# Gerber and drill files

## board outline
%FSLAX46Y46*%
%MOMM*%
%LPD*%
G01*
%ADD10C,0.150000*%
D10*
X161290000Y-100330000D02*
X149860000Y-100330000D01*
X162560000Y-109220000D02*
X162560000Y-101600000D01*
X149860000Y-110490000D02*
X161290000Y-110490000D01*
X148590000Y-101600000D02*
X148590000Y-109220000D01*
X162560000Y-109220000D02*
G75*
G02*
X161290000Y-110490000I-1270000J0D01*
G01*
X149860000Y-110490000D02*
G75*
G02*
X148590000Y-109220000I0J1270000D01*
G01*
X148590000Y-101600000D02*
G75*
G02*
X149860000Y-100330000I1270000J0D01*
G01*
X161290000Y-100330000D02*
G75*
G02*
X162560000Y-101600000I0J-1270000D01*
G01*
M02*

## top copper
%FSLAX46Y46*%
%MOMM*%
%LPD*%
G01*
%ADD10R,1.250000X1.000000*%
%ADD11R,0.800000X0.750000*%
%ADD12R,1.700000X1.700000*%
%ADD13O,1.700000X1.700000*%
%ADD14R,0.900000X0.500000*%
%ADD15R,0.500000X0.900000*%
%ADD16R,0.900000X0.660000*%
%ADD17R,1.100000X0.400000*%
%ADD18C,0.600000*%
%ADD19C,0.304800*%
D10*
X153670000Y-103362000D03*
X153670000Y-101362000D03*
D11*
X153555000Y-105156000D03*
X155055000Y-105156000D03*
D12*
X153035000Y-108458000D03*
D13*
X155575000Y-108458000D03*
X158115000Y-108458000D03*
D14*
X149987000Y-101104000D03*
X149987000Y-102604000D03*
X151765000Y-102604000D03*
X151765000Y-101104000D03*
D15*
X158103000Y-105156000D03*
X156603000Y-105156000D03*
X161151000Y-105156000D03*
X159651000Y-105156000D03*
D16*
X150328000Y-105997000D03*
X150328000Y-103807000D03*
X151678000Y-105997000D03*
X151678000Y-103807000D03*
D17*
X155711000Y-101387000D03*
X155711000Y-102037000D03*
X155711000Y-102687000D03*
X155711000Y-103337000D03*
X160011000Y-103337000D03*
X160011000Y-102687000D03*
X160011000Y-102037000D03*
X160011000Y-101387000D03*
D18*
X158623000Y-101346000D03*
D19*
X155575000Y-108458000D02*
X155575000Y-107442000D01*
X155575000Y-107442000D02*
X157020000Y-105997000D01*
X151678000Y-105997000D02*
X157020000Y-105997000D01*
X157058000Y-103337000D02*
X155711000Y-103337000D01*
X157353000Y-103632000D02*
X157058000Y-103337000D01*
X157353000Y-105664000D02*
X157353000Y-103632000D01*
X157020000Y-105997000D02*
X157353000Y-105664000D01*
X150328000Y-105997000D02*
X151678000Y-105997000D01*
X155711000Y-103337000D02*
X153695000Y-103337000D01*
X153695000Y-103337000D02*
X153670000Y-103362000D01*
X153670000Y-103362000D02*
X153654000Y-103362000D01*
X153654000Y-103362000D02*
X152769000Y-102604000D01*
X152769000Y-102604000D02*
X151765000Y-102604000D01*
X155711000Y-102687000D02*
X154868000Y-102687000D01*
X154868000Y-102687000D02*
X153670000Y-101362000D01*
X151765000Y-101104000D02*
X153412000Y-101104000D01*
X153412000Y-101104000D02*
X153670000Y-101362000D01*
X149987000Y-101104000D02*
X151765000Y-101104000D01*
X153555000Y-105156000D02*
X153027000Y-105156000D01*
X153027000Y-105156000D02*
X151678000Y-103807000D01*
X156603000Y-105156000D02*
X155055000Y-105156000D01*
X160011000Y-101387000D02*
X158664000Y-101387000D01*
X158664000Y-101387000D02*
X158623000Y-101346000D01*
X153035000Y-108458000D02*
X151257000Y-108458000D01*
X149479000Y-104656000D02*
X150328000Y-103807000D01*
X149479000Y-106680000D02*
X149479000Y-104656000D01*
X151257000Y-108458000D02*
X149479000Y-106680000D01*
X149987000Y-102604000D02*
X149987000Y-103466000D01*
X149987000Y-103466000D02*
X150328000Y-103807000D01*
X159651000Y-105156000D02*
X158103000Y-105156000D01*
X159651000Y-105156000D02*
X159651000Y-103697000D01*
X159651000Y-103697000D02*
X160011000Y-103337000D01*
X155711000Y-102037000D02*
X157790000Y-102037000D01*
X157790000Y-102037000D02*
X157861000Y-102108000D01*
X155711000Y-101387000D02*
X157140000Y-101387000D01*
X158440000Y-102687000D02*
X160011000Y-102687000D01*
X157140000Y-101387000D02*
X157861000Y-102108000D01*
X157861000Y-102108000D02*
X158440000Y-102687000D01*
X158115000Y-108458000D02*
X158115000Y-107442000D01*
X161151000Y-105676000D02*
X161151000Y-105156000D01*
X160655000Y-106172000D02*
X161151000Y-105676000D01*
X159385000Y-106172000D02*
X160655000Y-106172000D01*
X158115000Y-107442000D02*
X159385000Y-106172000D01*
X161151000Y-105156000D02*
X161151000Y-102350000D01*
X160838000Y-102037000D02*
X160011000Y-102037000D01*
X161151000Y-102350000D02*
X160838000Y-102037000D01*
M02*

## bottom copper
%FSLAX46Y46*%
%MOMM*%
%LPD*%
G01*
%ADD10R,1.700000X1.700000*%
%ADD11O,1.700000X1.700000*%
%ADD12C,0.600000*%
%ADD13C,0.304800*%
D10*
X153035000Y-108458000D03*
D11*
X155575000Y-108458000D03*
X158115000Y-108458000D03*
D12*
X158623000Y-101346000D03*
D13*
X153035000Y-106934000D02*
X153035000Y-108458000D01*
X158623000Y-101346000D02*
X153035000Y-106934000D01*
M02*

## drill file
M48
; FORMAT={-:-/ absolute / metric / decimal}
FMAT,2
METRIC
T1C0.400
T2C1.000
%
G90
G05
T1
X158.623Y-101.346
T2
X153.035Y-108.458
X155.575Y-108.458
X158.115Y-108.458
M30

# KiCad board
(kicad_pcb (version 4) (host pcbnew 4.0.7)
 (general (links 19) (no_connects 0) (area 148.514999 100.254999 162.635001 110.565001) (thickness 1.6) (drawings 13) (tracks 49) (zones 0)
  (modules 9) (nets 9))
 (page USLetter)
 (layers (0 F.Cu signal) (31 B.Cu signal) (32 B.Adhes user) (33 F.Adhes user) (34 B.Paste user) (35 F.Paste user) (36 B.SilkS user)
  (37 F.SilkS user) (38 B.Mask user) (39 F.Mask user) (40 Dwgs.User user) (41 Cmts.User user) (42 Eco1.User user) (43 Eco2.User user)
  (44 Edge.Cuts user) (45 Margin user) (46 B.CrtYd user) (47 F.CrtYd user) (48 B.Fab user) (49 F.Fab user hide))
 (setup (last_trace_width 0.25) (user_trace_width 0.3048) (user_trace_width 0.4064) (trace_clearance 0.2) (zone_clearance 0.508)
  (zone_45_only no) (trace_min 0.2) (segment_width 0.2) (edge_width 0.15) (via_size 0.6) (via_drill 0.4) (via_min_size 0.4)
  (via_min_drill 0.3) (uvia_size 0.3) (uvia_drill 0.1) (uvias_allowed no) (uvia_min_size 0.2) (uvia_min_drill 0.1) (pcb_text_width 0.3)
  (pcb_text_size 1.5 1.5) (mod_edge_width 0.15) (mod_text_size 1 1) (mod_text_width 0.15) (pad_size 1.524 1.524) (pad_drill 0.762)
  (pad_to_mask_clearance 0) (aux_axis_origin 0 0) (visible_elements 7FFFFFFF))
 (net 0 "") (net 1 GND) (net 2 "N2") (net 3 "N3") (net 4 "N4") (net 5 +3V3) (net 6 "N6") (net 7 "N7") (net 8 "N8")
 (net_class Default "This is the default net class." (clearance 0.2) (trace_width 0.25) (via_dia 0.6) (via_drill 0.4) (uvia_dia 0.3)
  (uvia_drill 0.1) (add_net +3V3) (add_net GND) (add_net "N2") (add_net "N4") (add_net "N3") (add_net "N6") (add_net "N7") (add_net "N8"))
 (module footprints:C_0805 (layer F.Cu) (at 153.67 102.362 90)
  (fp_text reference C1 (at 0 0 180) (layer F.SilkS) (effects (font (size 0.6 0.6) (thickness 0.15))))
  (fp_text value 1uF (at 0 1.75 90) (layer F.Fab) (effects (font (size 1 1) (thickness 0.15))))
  (pad 1 smd rect (at -1 0 90) (size 1 1.25) (layers F.Cu F.Paste F.Mask) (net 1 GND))
  (pad 2 smd rect (at 1 0 90) (size 1 1.25) (layers F.Cu F.Paste F.Mask) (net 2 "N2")))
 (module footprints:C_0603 (layer F.Cu) (at 154.305 105.156 180)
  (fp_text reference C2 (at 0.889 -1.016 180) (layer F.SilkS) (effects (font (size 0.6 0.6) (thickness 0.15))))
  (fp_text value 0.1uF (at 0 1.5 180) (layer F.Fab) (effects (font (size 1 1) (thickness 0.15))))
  (pad 2 smd rect (at 0.75 0 180) (size 0.8 0.75) (layers F.Cu F.Paste F.Mask) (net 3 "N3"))
  (pad 1 smd rect (at -0.75 0 180) (size 0.8 0.75) (layers F.Cu F.Paste F.Mask) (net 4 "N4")))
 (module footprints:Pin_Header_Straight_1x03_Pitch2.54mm (layer F.Cu) (at 153.035 108.458 90)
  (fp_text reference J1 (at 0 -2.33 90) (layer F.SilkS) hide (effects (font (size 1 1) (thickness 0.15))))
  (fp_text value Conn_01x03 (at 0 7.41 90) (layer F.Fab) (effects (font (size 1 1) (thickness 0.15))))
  (pad 1 thru_hole rect (at 0 0 90) (size 1.7 1.7) (drill 1) (layers *.Cu *.Mask) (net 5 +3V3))
  (pad 2 thru_hole oval (at 0 2.54 90) (size 1.7 1.7) (drill 1) (layers *.Cu *.Mask) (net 1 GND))
  (pad 3 thru_hole oval (at 0 5.08 90) (size 1.7 1.7) (drill 1) (layers *.Cu *.Mask) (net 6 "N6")))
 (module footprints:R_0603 (layer F.Cu) (at 149.987 101.854 270)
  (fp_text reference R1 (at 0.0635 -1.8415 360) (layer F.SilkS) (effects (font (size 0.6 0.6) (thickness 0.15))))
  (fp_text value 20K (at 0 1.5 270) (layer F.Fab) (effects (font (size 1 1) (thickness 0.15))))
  (pad 1 smd rect (at -0.75 0 270) (size 0.5 0.9) (layers F.Cu F.Paste F.Mask) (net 2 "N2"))
  (pad 2 smd rect (at 0.75 0 270) (size 0.5 0.9) (layers F.Cu F.Paste F.Mask) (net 5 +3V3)))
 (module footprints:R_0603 (layer F.Cu) (at 151.765 101.854 90)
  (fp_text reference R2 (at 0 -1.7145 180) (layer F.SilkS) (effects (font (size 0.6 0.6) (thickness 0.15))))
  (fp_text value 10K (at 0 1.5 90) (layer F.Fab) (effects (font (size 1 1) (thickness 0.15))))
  (pad 1 smd rect (at -0.75 0 90) (size 0.5 0.9) (layers F.Cu F.Paste F.Mask) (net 1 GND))
  (pad 2 smd rect (at 0.75 0 90) (size 0.5 0.9) (layers F.Cu F.Paste F.Mask) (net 2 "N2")))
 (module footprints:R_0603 (layer F.Cu) (at 157.353 105.156 180)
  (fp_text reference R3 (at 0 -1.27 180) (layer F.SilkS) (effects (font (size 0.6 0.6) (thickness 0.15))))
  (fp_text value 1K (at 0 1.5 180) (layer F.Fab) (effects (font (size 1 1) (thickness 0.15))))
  (pad 1 smd rect (at -0.75 0 180) (size 0.5 0.9) (layers F.Cu F.Paste F.Mask) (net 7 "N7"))
  (pad 2 smd rect (at 0.75 0 180) (size 0.5 0.9) (layers F.Cu F.Paste F.Mask) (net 4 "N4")))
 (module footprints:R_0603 (layer F.Cu) (at 160.401 105.156 180)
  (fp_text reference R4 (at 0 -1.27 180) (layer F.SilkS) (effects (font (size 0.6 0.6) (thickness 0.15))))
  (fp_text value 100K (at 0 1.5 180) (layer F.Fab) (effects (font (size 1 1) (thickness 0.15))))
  (pad 1 smd rect (at -0.75 0 180) (size 0.5 0.9) (layers F.Cu F.Paste F.Mask) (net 6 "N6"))
  (pad 2 smd rect (at 0.75 0 180) (size 0.5 0.9) (layers F.Cu F.Paste F.Mask) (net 7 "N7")))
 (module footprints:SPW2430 (layer F.Cu) (at 151.003 104.902)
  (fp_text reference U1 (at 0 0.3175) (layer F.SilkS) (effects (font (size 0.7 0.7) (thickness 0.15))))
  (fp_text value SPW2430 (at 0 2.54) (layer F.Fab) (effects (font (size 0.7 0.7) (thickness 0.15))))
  (pad 3 smd rect (at -0.675 1.095) (size 0.9 0.66) (layers F.Cu F.Paste F.Mask) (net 1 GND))
  (pad 4 smd rect (at -0.675 -1.095) (size 0.9 0.66) (layers F.Cu F.Paste F.Mask) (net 5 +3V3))
  (pad 2 smd rect (at 0.675 1.095) (size 0.9 0.66) (layers F.Cu F.Paste F.Mask) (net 1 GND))
  (pad 1 smd rect (at 0.675 -1.095) (size 0.9 0.66) (layers F.Cu F.Paste F.Mask) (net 3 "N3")))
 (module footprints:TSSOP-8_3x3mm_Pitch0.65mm (layer F.Cu) (at 157.861 102.362)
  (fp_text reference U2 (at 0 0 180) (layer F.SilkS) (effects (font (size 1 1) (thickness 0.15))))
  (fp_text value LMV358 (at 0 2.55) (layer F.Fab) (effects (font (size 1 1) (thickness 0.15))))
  (pad 1 smd rect (at -2.15 -0.975) (size 1.1 0.4) (layers F.Cu F.Paste F.Mask) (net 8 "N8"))
  (pad 2 smd rect (at -2.15 -0.325) (size 1.1 0.4) (layers F.Cu F.Paste F.Mask) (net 8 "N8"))
  (pad 3 smd rect (at -2.15 0.325) (size 1.1 0.4) (layers F.Cu F.Paste F.Mask) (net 2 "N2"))
  (pad 4 smd rect (at -2.15 0.975) (size 1.1 0.4) (layers F.Cu F.Paste F.Mask) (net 1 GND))
  (pad 5 smd rect (at 2.15 0.975) (size 1.1 0.4) (layers F.Cu F.Paste F.Mask) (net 7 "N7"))
  (pad 6 smd rect (at 2.15 0.325) (size 1.1 0.4) (layers F.Cu F.Paste F.Mask) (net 8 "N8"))
  (pad 7 smd rect (at 2.15 -0.325) (size 1.1 0.4) (layers F.Cu F.Paste F.Mask) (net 6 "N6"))
  (pad 8 smd rect (at 2.15 -0.975) (size 1.1 0.4) (layers F.Cu F.Paste F.Mask) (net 5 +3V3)))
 (gr_line (start 161.29 100.33) (end 149.86 100.33) (angle 90) (layer Edge.Cuts) (width 0.15))
 (gr_line (start 162.56 109.22) (end 162.56 101.6) (angle 90) (layer Edge.Cuts) (width 0.15))
 (gr_line (start 149.86 110.49) (end 161.29 110.49) (angle 90) (layer Edge.Cuts) (width 0.15))
 (gr_line (start 148.59 101.6) (end 148.59 109.22) (angle 90) (layer Edge.Cuts) (width 0.15))
 (gr_arc (start 161.29 109.22) (end 162.56 109.22) (angle 90) (layer Edge.Cuts) (width 0.15))
 (gr_arc (start 149.86 109.22) (end 149.86 110.49) (angle 90) (layer Edge.Cuts) (width 0.15))
 (gr_arc (start 149.86 101.6) (end 148.59 101.6) (angle 90) (layer Edge.Cuts) (width 0.15))
 (gr_arc (start 161.29 101.6) (end 161.29 100.33) (angle 90) (layer Edge.Cuts) (width 0.15))
 (segment (start 155.575 108.458) (end 155.575 107.442) (width 0.3048) (layer F.Cu) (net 1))
 (segment (start 155.575 107.442) (end 157.02 105.997) (width 0.3048) (layer F.Cu) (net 1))
 (segment (start 151.678 105.997) (end 157.02 105.997) (width 0.3048) (layer F.Cu) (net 1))
 (segment (start 157.058 103.337) (end 155.711 103.337) (width 0.3048) (layer F.Cu) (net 1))
 (segment (start 157.353 103.632) (end 157.058 103.337) (width 0.3048) (layer F.Cu) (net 1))
 (segment (start 157.353 105.664) (end 157.353 103.632) (width 0.3048) (layer F.Cu) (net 1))
 (segment (start 157.02 105.997) (end 157.353 105.664) (width 0.3048) (layer F.Cu) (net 1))
 (segment (start 150.328 105.997) (end 151.678 105.997) (width 0.3048) (layer F.Cu) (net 1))
 (segment (start 155.711 103.337) (end 153.695 103.337) (width 0.3048) (layer F.Cu) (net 1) (status 20))
 (segment (start 153.695 103.337) (end 153.67 103.362) (width 0.3048) (layer F.Cu) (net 1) (status 30))
 (segment (start 153.67 103.362) (end 153.654 103.362) (width 0.3048) (layer F.Cu) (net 1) (status 30))
 (segment (start 153.654 103.362) (end 152.769 102.604) (width 0.3048) (layer F.Cu) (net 1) (status 10))
 (segment (start 152.769 102.604) (end 151.765 102.604) (width 0.3048) (layer F.Cu) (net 1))
 (segment (start 155.711 102.687) (end 154.868 102.687) (width 0.3048) (layer F.Cu) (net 2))
 (segment (start 154.868 102.687) (end 153.67 101.362) (width 0.3048) (layer F.Cu) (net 2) (status 20))
 (segment (start 151.765 101.104) (end 153.412 101.104) (width 0.3048) (layer F.Cu) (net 2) (status 20))
 (segment (start 153.412 101.104) (end 153.67 101.362) (width 0.3048) (layer F.Cu) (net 2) (status 30))
 (segment (start 149.987 101.104) (end 151.765 101.104) (width 0.3048) (layer F.Cu) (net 2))
 (segment (start 153.555 105.156) (end 153.027 105.156) (width 0.3048) (layer F.Cu) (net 3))
 (segment (start 153.027 105.156) (end 151.678 103.807) (width 0.3048) (layer F.Cu) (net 3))
 (segment (start 156.603 105.156) (end 155.055 105.156) (width 0.3048) (layer F.Cu) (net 4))
 (segment (start 160.011 101.387) (end 158.664 101.387) (width 0.3048) (layer F.Cu) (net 5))
 (segment (start 153.035 106.934) (end 153.035 108.458) (width 0.3048) (layer B.Cu) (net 5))
 (segment (start 158.623 101.346) (end 153.035 106.934) (width 0.3048) (layer B.Cu) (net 5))
 (via (at 158.623 101.346) (size 0.6) (drill 0.4) (layers F.Cu B.Cu) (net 5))
 (segment (start 158.664 101.387) (end 158.623 101.346) (width 0.3048) (layer F.Cu) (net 5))
 (segment (start 153.035 108.458) (end 151.257 108.458) (width 0.3048) (layer F.Cu) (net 5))
 (segment (start 149.479 104.656) (end 150.328 103.807) (width 0.3048) (layer F.Cu) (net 5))
 (segment (start 149.479 106.68) (end 149.479 104.656) (width 0.3048) (layer F.Cu) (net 5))
 (segment (start 151.257 108.458) (end 149.479 106.68) (width 0.3048) (layer F.Cu) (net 5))
 (segment (start 149.987 102.604) (end 149.987 103.466) (width 0.3048) (layer F.Cu) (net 5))
 (segment (start 149.987 103.466) (end 150.328 103.807) (width 0.3048) (layer F.Cu) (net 5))
 (segment (start 159.651 105.156) (end 158.103 105.156) (width 0.3048) (layer F.Cu) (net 7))
 (segment (start 159.651 105.156) (end 159.651 103.697) (width 0.3048) (layer F.Cu) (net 7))
 (segment (start 159.651 103.697) (end 160.011 103.337) (width 0.3048) (layer F.Cu) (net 7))
 (segment (start 155.711 102.037) (end 157.79 102.037) (width 0.3048) (layer F.Cu) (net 8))
 (segment (start 157.79 102.037) (end 157.861 102.108) (width 0.3048) (layer F.Cu) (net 8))
 (segment (start 155.711 101.387) (end 157.14 101.387) (width 0.3048) (layer F.Cu) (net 8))
 (segment (start 158.44 102.687) (end 160.011 102.687) (width 0.3048) (layer F.Cu) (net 8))
 (segment (start 157.14 101.387) (end 157.861 102.108) (width 0.3048) (layer F.Cu) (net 8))
 (segment (start 157.861 102.108) (end 158.44 102.687) (width 0.3048) (layer F.Cu) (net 8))
 (segment (start 158.115 108.458) (end 158.115 107.442) (width 0.3048) (layer F.Cu) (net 6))
 (segment (start 161.151 105.676) (end 161.151 105.156) (width 0.3048) (layer F.Cu) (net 6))
 (segment (start 160.655 106.172) (end 161.151 105.676) (width 0.3048) (layer F.Cu) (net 6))
 (segment (start 159.385 106.172) (end 160.655 106.172) (width 0.3048) (layer F.Cu) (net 6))
 (segment (start 158.115 107.442) (end 159.385 106.172) (width 0.3048) (layer F.Cu) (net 6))
 (segment (start 161.151 105.156) (end 161.151 102.35) (width 0.3048) (layer F.Cu) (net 6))
 (segment (start 160.838 102.037) (end 160.011 102.037) (width 0.3048) (layer F.Cu) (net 6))
 (segment (start 161.151 102.35) (end 160.838 102.037) (width 0.3048) (layer F.Cu) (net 6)))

